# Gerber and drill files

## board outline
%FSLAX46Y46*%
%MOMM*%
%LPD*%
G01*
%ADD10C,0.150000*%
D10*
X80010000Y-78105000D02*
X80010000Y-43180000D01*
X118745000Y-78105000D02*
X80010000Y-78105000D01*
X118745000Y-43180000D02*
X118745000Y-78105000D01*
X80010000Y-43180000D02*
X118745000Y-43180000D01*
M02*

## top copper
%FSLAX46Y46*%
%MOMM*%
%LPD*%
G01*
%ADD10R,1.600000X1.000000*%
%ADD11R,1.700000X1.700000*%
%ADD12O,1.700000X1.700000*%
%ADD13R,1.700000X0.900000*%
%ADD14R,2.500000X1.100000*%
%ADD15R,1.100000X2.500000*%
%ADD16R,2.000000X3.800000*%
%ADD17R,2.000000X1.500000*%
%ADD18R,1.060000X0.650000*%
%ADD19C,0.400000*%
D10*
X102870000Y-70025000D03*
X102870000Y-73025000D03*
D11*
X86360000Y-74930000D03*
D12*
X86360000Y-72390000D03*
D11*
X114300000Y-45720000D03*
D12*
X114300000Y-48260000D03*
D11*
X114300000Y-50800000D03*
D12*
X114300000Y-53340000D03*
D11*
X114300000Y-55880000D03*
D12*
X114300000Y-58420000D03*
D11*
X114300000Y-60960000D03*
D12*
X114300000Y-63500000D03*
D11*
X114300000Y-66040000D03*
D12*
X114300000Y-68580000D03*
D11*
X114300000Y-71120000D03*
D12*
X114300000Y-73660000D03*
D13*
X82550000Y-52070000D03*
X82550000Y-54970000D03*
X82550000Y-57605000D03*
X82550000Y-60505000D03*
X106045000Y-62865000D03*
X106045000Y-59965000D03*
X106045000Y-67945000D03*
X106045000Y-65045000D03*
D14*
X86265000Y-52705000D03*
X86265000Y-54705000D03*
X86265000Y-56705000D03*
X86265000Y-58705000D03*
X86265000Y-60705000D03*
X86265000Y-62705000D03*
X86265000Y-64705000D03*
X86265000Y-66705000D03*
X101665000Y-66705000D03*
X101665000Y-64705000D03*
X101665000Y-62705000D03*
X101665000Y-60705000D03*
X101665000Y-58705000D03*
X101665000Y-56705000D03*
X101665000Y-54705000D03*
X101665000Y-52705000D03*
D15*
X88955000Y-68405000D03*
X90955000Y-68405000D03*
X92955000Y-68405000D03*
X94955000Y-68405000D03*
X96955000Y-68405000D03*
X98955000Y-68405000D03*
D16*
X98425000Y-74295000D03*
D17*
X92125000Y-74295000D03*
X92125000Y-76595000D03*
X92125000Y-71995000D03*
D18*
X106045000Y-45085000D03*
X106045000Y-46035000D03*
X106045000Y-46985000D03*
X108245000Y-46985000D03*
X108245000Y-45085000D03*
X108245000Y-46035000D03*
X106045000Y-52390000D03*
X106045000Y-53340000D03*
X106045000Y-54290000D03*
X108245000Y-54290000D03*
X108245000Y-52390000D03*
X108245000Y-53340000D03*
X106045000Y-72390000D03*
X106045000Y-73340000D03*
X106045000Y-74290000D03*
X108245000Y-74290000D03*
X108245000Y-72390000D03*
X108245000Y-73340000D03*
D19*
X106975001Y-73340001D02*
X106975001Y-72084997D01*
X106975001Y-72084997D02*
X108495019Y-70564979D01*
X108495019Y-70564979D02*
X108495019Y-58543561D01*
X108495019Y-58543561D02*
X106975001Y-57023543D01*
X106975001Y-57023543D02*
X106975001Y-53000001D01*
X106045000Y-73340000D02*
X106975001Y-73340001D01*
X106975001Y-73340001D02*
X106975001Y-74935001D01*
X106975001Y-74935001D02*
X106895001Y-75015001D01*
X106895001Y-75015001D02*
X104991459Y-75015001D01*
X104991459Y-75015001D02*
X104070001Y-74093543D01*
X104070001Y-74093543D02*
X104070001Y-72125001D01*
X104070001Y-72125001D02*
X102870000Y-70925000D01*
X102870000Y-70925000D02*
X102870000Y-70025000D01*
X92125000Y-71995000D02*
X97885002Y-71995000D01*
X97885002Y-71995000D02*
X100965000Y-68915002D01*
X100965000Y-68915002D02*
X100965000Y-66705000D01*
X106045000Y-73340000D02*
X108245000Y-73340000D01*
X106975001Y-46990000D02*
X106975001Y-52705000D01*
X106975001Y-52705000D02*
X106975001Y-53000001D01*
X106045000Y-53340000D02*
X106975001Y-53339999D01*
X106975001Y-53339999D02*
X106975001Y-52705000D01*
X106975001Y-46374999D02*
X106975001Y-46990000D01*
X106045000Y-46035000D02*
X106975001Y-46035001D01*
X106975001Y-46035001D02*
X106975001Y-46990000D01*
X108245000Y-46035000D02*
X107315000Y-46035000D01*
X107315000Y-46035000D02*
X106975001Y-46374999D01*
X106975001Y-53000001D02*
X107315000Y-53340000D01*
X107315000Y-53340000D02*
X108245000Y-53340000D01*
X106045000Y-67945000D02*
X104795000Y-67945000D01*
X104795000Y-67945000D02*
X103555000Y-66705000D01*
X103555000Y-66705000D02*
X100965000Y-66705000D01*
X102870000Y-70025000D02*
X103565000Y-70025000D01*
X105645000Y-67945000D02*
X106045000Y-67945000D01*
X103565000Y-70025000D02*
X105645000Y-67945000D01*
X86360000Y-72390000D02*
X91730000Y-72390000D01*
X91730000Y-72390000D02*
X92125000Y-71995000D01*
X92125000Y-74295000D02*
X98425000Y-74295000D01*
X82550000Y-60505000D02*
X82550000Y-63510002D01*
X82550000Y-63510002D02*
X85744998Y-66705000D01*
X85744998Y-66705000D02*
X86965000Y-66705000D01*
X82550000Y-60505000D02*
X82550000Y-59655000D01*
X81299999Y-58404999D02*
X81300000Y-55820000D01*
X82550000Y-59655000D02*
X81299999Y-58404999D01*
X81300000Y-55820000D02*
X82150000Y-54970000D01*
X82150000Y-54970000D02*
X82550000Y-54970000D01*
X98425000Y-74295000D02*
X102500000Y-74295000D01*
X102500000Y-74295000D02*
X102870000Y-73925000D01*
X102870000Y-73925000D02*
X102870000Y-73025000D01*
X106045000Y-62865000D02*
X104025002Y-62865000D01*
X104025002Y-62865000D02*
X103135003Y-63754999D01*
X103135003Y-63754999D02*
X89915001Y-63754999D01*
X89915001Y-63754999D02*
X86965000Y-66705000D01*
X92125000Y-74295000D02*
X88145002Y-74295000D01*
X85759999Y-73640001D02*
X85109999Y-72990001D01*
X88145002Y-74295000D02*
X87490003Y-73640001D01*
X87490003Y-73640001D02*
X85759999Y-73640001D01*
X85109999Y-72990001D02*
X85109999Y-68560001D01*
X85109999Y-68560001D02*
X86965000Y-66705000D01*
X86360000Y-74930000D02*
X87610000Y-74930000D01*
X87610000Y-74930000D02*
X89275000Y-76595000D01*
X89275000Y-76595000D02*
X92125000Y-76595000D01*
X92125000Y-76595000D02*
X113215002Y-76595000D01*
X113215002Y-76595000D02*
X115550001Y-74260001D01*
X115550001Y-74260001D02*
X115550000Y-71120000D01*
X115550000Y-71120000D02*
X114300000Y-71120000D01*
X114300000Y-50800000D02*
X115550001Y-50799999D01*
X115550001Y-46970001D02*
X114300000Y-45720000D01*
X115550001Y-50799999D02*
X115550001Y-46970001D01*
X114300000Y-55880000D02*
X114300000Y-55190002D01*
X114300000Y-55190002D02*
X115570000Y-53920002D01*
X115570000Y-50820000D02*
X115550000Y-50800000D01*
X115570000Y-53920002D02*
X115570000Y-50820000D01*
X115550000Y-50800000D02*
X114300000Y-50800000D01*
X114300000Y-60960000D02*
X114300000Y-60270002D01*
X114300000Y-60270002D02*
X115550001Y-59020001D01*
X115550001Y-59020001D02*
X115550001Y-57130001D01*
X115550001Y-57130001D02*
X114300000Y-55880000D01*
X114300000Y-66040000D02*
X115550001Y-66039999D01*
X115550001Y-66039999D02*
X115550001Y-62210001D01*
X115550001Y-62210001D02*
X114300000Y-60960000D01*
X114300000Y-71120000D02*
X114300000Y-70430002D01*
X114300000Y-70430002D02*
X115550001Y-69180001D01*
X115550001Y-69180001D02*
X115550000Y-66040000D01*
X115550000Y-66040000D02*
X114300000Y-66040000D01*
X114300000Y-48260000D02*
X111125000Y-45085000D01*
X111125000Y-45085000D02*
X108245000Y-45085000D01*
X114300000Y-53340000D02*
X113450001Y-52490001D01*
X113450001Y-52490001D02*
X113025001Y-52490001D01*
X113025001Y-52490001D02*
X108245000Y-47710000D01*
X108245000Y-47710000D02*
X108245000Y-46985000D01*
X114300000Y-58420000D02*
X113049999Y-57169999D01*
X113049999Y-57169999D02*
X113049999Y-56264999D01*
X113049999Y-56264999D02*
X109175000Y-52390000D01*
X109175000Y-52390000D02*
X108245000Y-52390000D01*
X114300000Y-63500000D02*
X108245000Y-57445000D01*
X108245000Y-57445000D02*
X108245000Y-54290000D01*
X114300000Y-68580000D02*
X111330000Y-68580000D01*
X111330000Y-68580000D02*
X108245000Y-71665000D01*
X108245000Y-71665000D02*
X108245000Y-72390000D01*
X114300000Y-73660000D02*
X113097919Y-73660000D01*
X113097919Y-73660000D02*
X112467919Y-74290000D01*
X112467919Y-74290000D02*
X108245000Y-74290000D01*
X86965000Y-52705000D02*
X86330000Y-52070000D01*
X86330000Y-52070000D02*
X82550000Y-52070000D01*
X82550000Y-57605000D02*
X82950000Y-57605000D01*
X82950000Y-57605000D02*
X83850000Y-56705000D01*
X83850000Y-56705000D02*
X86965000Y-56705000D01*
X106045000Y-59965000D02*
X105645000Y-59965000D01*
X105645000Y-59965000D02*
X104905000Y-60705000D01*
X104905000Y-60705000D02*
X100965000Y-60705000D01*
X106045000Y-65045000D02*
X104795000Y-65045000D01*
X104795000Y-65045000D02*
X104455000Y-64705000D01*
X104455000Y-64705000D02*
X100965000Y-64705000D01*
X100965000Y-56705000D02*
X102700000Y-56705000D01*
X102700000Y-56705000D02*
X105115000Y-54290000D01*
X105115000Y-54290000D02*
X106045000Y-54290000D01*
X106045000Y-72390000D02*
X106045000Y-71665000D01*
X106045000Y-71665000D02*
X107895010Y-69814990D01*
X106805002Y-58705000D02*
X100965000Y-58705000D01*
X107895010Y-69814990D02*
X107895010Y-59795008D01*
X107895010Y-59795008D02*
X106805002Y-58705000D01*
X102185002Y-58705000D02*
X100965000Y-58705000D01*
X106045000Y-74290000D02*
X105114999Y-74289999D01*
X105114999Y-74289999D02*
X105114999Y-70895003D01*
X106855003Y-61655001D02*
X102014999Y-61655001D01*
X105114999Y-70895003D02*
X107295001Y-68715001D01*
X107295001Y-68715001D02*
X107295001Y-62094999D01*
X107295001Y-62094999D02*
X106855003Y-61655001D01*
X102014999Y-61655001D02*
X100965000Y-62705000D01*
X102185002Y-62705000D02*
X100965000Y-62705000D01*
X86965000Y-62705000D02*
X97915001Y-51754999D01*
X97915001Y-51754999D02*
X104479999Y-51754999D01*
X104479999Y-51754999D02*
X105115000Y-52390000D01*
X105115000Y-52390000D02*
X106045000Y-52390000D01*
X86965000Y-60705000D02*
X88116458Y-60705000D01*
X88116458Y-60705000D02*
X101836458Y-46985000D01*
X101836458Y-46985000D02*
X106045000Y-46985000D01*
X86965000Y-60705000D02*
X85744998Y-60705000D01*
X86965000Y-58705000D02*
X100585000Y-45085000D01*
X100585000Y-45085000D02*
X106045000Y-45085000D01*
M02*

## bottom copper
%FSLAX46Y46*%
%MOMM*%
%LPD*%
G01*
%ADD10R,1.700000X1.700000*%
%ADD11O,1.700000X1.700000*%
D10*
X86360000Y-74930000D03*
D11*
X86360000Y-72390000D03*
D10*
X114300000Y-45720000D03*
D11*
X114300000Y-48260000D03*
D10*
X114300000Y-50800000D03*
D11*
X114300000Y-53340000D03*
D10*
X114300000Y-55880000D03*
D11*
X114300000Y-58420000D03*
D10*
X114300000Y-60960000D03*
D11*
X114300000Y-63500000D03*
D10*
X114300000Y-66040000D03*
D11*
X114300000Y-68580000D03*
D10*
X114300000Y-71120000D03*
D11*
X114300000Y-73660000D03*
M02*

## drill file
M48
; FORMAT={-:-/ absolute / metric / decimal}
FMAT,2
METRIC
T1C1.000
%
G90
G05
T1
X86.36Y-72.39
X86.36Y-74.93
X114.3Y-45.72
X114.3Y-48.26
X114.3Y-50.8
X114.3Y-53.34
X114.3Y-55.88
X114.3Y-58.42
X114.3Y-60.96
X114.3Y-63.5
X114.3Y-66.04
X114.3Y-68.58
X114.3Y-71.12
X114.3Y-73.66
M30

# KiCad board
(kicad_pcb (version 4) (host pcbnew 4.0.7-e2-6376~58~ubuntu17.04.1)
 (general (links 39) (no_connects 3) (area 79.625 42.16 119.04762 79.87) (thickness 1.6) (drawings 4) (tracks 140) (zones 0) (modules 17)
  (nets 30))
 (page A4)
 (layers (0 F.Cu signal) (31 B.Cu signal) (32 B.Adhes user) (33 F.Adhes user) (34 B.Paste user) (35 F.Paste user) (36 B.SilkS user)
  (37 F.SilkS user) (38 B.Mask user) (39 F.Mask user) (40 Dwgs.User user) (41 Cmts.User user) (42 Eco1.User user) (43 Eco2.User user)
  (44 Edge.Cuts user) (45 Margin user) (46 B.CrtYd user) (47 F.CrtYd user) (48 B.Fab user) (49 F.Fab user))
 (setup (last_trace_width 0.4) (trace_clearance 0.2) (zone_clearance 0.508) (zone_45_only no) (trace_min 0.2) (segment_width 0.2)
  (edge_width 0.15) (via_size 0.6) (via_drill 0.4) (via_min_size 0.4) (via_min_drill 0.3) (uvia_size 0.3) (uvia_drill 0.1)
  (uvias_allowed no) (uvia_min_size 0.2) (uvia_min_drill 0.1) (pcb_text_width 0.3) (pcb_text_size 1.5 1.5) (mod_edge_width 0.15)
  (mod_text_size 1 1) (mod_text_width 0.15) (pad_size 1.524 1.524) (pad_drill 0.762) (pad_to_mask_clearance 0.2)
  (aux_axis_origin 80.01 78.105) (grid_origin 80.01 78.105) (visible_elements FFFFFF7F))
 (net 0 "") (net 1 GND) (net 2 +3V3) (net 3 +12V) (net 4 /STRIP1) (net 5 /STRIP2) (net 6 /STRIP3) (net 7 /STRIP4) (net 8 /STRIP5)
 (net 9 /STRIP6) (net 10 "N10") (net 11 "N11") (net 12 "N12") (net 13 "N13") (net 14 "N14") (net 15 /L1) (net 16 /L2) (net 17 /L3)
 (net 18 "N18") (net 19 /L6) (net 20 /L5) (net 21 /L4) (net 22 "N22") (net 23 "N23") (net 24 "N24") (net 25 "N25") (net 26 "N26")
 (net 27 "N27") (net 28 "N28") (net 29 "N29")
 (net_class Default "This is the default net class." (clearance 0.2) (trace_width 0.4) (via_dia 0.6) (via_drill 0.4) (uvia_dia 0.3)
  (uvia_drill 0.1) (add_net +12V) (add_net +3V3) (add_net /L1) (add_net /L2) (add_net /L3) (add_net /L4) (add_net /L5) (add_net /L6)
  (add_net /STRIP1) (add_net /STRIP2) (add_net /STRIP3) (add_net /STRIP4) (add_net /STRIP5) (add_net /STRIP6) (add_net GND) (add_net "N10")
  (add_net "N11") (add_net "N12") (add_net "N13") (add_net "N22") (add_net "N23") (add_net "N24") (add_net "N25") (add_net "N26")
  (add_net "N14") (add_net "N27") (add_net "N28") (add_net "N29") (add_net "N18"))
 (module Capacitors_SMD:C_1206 (layer F.Cu) (at 102.87 71.525 270)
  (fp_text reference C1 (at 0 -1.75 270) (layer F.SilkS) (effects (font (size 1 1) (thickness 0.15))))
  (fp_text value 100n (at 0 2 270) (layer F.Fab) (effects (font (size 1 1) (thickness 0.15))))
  (pad 1 smd rect (at -1.5 0 270) (size 1 1.6) (layers F.Cu F.Paste F.Mask) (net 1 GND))
  (pad 2 smd rect (at 1.5 0 270) (size 1 1.6) (layers F.Cu F.Paste F.Mask) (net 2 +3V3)))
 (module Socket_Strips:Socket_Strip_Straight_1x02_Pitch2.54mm (layer F.Cu) (at 86.36 74.93 180)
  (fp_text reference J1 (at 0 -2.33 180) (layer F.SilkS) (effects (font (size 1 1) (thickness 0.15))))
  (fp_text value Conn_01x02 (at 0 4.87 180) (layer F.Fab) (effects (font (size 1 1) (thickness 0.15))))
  (pad 1 thru_hole rect (at 0 0 180) (size 1.7 1.7) (drill 1) (layers *.Cu *.Mask) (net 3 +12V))
  (pad 2 thru_hole oval (at 0 2.54 180) (size 1.7 1.7) (drill 1) (layers *.Cu *.Mask) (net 1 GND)))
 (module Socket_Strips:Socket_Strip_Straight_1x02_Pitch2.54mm (layer F.Cu) (at 114.3 45.72)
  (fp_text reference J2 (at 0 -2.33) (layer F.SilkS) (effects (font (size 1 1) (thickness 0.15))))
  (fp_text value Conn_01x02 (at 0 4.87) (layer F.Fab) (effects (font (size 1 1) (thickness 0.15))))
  (pad 1 thru_hole rect (at 0 0) (size 1.7 1.7) (drill 1) (layers *.Cu *.Mask) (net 3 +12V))
  (pad 2 thru_hole oval (at 0 2.54) (size 1.7 1.7) (drill 1) (layers *.Cu *.Mask) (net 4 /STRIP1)))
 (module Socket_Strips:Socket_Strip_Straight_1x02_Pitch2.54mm (layer F.Cu) (at 114.3 50.8)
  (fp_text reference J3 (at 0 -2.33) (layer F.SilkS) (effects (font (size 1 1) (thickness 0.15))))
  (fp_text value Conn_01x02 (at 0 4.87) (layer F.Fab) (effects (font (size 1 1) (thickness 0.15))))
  (pad 1 thru_hole rect (at 0 0) (size 1.7 1.7) (drill 1) (layers *.Cu *.Mask) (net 3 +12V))
  (pad 2 thru_hole oval (at 0 2.54) (size 1.7 1.7) (drill 1) (layers *.Cu *.Mask) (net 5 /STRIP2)))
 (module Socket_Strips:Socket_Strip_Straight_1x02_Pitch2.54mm (layer F.Cu) (at 114.3 55.88)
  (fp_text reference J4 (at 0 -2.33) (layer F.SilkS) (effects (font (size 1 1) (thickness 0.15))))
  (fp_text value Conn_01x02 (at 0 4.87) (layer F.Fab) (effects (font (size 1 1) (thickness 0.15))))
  (pad 1 thru_hole rect (at 0 0) (size 1.7 1.7) (drill 1) (layers *.Cu *.Mask) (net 3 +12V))
  (pad 2 thru_hole oval (at 0 2.54) (size 1.7 1.7) (drill 1) (layers *.Cu *.Mask) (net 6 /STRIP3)))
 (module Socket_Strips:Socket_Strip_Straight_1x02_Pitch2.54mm (layer F.Cu) (at 114.3 60.96)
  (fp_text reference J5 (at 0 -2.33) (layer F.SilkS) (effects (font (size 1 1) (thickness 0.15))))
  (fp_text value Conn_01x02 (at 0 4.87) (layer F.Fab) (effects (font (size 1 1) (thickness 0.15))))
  (pad 1 thru_hole rect (at 0 0) (size 1.7 1.7) (drill 1) (layers *.Cu *.Mask) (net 3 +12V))
  (pad 2 thru_hole oval (at 0 2.54) (size 1.7 1.7) (drill 1) (layers *.Cu *.Mask) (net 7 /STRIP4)))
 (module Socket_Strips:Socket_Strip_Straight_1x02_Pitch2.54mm (layer F.Cu) (at 114.3 66.04)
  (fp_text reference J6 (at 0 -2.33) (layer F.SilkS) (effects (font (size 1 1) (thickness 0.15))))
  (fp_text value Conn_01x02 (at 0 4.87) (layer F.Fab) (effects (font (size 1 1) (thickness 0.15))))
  (pad 1 thru_hole rect (at 0 0) (size 1.7 1.7) (drill 1) (layers *.Cu *.Mask) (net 3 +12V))
  (pad 2 thru_hole oval (at 0 2.54) (size 1.7 1.7) (drill 1) (layers *.Cu *.Mask) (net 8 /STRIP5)))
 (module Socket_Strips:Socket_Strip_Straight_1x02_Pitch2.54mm (layer F.Cu) (at 114.3 71.12)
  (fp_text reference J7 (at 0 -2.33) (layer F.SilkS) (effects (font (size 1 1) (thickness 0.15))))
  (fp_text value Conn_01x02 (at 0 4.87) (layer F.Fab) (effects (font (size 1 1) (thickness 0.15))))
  (pad 1 thru_hole rect (at 0 0) (size 1.7 1.7) (drill 1) (layers *.Cu *.Mask) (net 3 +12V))
  (pad 2 thru_hole oval (at 0 2.54) (size 1.7 1.7) (drill 1) (layers *.Cu *.Mask) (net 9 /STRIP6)))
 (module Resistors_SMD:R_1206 (layer F.Cu) (at 82.55 53.52 270)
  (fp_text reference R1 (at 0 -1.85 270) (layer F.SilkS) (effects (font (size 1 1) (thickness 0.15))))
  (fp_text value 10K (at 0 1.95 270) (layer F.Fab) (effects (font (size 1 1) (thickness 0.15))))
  (pad 1 smd rect (at -1.45 0 270) (size 0.9 1.7) (layers F.Cu F.Paste F.Mask) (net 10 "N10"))
  (pad 2 smd rect (at 1.45 0 270) (size 0.9 1.7) (layers F.Cu F.Paste F.Mask) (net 2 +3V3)))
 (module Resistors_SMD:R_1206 (layer F.Cu) (at 82.55 59.055 270)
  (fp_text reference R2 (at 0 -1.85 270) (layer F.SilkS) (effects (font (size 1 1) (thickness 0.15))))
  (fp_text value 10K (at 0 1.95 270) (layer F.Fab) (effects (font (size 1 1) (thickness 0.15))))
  (pad 1 smd rect (at -1.45 0 270) (size 0.9 1.7) (layers F.Cu F.Paste F.Mask) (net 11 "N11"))
  (pad 2 smd rect (at 1.45 0 270) (size 0.9 1.7) (layers F.Cu F.Paste F.Mask) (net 2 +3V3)))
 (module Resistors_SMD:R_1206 (layer F.Cu) (at 106.045 61.415 90)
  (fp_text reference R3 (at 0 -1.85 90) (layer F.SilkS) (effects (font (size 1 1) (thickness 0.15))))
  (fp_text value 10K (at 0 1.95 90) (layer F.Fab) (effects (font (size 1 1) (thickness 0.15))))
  (pad 1 smd rect (at -1.45 0 90) (size 0.9 1.7) (layers F.Cu F.Paste F.Mask) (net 2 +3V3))
  (pad 2 smd rect (at 1.45 0 90) (size 0.9 1.7) (layers F.Cu F.Paste F.Mask) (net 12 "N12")))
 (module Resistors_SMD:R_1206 (layer F.Cu) (at 106.045 66.495 90)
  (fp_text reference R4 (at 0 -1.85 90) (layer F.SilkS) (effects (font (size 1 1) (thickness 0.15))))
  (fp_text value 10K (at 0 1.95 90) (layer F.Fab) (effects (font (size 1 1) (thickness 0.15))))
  (pad 1 smd rect (at -1.45 0 90) (size 0.9 1.7) (layers F.Cu F.Paste F.Mask) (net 1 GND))
  (pad 2 smd rect (at 1.45 0 90) (size 0.9 1.7) (layers F.Cu F.Paste F.Mask) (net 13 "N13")))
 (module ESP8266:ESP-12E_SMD (layer F.Cu) (at 86.965 52.705)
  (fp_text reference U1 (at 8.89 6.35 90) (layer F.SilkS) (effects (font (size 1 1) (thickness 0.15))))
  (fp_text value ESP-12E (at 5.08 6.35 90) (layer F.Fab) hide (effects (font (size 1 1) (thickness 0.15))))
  (pad 1 smd rect (at 0 0) (size 2.5 1.1) (drill (offset -0.7 0)) (layers F.Cu F.Paste F.Mask) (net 10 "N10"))
  (pad 2 smd rect (at 0 2) (size 2.5 1.1) (drill (offset -0.7 0)) (layers F.Cu F.Paste F.Mask) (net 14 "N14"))
  (pad 3 smd rect (at 0 4) (size 2.5 1.1) (drill (offset -0.7 0)) (layers F.Cu F.Paste F.Mask) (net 11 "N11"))
  (pad 4 smd rect (at 0 6) (size 2.5 1.1) (drill (offset -0.7 0)) (layers F.Cu F.Paste F.Mask) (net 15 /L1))
  (pad 5 smd rect (at 0 8) (size 2.5 1.1) (drill (offset -0.7 0)) (layers F.Cu F.Paste F.Mask) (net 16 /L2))
  (pad 6 smd rect (at 0 10) (size 2.5 1.1) (drill (offset -0.7 0)) (layers F.Cu F.Paste F.Mask) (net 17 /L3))
  (pad 7 smd rect (at 0 12) (size 2.5 1.1) (drill (offset -0.7 0)) (layers F.Cu F.Paste F.Mask) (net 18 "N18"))
  (pad 8 smd rect (at 0 14) (size 2.5 1.1) (drill (offset -0.7 0)) (layers F.Cu F.Paste F.Mask) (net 2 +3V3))
  (pad 9 smd rect (at 14 14) (size 2.5 1.1) (drill (offset 0.7 0)) (layers F.Cu F.Paste F.Mask) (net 1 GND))
  (pad 10 smd rect (at 14 12) (size 2.5 1.1) (drill (offset 0.7 0)) (layers F.Cu F.Paste F.Mask) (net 13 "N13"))
  (pad 11 smd rect (at 14 10) (size 2.5 1.1) (drill (offset 0.7 0)) (layers F.Cu F.Paste F.Mask) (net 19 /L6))
  (pad 12 smd rect (at 14 8) (size 2.5 1.1) (drill (offset 0.7 0)) (layers F.Cu F.Paste F.Mask) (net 12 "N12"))
  (pad 13 smd rect (at 14 6) (size 2.5 1.1) (drill (offset 0.7 0)) (layers F.Cu F.Paste F.Mask) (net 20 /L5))
  (pad 14 smd rect (at 14 4) (size 2.5 1.1) (drill (offset 0.7 0)) (layers F.Cu F.Paste F.Mask) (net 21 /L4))
  (pad 15 smd rect (at 14 2) (size 2.5 1.1) (drill (offset 0.7 0)) (layers F.Cu F.Paste F.Mask) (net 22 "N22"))
  (pad 16 smd rect (at 14 0) (size 2.5 1.1) (drill (offset 0.7 0)) (layers F.Cu F.Paste F.Mask) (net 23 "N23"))
  (pad 17 smd rect (at 1.99 15 90) (size 2.5 1.1) (drill (offset -0.7 0)) (layers F.Cu F.Paste F.Mask) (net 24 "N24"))
  (pad 18 smd rect (at 3.99 15 90) (size 2.5 1.1) (drill (offset -0.7 0)) (layers F.Cu F.Paste F.Mask) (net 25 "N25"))
  (pad 19 smd rect (at 5.99 15 90) (size 2.5 1.1) (drill (offset -0.7 0)) (layers F.Cu F.Paste F.Mask) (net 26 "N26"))
  (pad 20 smd rect (at 7.99 15 90) (size 2.5 1.1) (drill (offset -0.7 0)) (layers F.Cu F.Paste F.Mask) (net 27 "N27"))
  (pad 21 smd rect (at 9.99 15 90) (size 2.5 1.1) (drill (offset -0.7 0)) (layers F.Cu F.Paste F.Mask) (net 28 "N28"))
  (pad 22 smd rect (at 11.99 15 90) (size 2.5 1.1) (drill (offset -0.7 0)) (layers F.Cu F.Paste F.Mask) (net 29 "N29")))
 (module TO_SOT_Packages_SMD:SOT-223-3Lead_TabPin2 (layer F.Cu) (at 95.275 74.295)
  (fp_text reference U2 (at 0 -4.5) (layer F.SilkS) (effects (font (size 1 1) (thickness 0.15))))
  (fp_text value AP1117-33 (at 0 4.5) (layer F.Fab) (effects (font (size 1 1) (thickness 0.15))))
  (pad 2 smd rect (at 3.15 0) (size 2 3.8) (layers F.Cu F.Paste F.Mask) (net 2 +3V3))
  (pad 2 smd rect (at -3.15 0) (size 2 1.5) (layers F.Cu F.Paste F.Mask) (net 2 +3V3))
  (pad 3 smd rect (at -3.15 2.3) (size 2 1.5) (layers F.Cu F.Paste F.Mask) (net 3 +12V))
  (pad 1 smd rect (at -3.15 -2.3) (size 2 1.5) (layers F.Cu F.Paste F.Mask) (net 1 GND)))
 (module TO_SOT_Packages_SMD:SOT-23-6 (layer F.Cu) (at 107.145 46.035)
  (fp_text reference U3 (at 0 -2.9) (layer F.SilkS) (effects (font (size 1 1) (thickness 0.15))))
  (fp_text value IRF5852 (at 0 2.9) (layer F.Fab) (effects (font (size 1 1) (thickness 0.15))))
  (pad 1 smd rect (at -1.1 -0.95) (size 1.06 0.65) (layers F.Cu F.Paste F.Mask) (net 15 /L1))
  (pad 2 smd rect (at -1.1 0) (size 1.06 0.65) (layers F.Cu F.Paste F.Mask) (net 1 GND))
  (pad 3 smd rect (at -1.1 0.95) (size 1.06 0.65) (layers F.Cu F.Paste F.Mask) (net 16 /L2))
  (pad 4 smd rect (at 1.1 0.95) (size 1.06 0.65) (layers F.Cu F.Paste F.Mask) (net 5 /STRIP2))
  (pad 6 smd rect (at 1.1 -0.95) (size 1.06 0.65) (layers F.Cu F.Paste F.Mask) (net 4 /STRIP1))
  (pad 5 smd rect (at 1.1 0) (size 1.06 0.65) (layers F.Cu F.Paste F.Mask) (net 1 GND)))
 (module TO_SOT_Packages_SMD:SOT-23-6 (layer F.Cu) (at 107.145 53.34)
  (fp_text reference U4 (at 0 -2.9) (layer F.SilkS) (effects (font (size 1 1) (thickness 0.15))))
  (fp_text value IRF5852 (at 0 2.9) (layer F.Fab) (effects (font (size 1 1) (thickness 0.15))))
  (pad 1 smd rect (at -1.1 -0.95) (size 1.06 0.65) (layers F.Cu F.Paste F.Mask) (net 17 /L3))
  (pad 2 smd rect (at -1.1 0) (size 1.06 0.65) (layers F.Cu F.Paste F.Mask) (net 1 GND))
  (pad 3 smd rect (at -1.1 0.95) (size 1.06 0.65) (layers F.Cu F.Paste F.Mask) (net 21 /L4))
  (pad 4 smd rect (at 1.1 0.95) (size 1.06 0.65) (layers F.Cu F.Paste F.Mask) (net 7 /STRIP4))
  (pad 6 smd rect (at 1.1 -0.95) (size 1.06 0.65) (layers F.Cu F.Paste F.Mask) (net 6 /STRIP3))
  (pad 5 smd rect (at 1.1 0) (size 1.06 0.65) (layers F.Cu F.Paste F.Mask) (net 1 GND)))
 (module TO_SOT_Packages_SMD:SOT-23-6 (layer F.Cu) (at 107.145 73.34)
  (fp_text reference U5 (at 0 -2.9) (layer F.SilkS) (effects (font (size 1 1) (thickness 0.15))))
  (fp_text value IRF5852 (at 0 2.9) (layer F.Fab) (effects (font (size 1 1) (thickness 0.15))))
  (pad 1 smd rect (at -1.1 -0.95) (size 1.06 0.65) (layers F.Cu F.Paste F.Mask) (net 20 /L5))
  (pad 2 smd rect (at -1.1 0) (size 1.06 0.65) (layers F.Cu F.Paste F.Mask) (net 1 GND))
  (pad 3 smd rect (at -1.1 0.95) (size 1.06 0.65) (layers F.Cu F.Paste F.Mask) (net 19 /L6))
  (pad 4 smd rect (at 1.1 0.95) (size 1.06 0.65) (layers F.Cu F.Paste F.Mask) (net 9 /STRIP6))
  (pad 6 smd rect (at 1.1 -0.95) (size 1.06 0.65) (layers F.Cu F.Paste F.Mask) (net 8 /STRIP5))
  (pad 5 smd rect (at 1.1 0) (size 1.06 0.65) (layers F.Cu F.Paste F.Mask) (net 1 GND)))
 (gr_line (start 80.01 78.105) (end 80.01 43.18) (layer Edge.Cuts) (width 0.15))
 (gr_line (start 118.745 78.105) (end 80.01 78.105) (layer Edge.Cuts) (width 0.15))
 (gr_line (start 118.745 43.18) (end 118.745 78.105) (layer Edge.Cuts) (width 0.15))
 (gr_line (start 80.01 43.18) (end 118.745 43.18) (layer Edge.Cuts) (width 0.15))
 (segment (start 106.975001 73.340001) (end 106.975001 72.084997) (width 0.4) (layer F.Cu) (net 1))
 (segment (start 106.975001 72.084997) (end 108.495019 70.564979) (width 0.4) (layer F.Cu) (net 1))
 (segment (start 108.495019 70.564979) (end 108.495019 58.543561) (width 0.4) (layer F.Cu) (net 1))
 (segment (start 108.495019 58.543561) (end 106.975001 57.023543) (width 0.4) (layer F.Cu) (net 1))
 (segment (start 106.975001 57.023543) (end 106.975001 53.000001) (width 0.4) (layer F.Cu) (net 1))
 (segment (start 106.045 73.34) (end 106.975001 73.340001) (width 0.4) (layer F.Cu) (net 1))
 (segment (start 106.975001 73.340001) (end 106.975001 74.935001) (width 0.4) (layer F.Cu) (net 1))
 (segment (start 106.975001 74.935001) (end 106.895001 75.015001) (width 0.4) (layer F.Cu) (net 1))
 (segment (start 106.895001 75.015001) (end 104.991459 75.015001) (width 0.4) (layer F.Cu) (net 1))
 (segment (start 104.991459 75.015001) (end 104.070001 74.093543) (width 0.4) (layer F.Cu) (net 1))
 (segment (start 104.070001 74.093543) (end 104.070001 72.125001) (width 0.4) (layer F.Cu) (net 1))
 (segment (start 104.070001 72.125001) (end 102.87 70.925) (width 0.4) (layer F.Cu) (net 1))
 (segment (start 102.87 70.925) (end 102.87 70.025) (width 0.4) (layer F.Cu) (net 1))
 (segment (start 92.125 71.995) (end 97.885002 71.995) (width 0.4) (layer F.Cu) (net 1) (status 10))
 (segment (start 97.885002 71.995) (end 100.965 68.915002) (width 0.4) (layer F.Cu) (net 1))
 (segment (start 100.965 68.915002) (end 100.965 66.705) (width 0.4) (layer F.Cu) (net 1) (status 20))
 (segment (start 106.045 73.34) (end 108.245 73.34) (width 0.4) (layer F.Cu) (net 1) (status 30))
 (segment (start 106.975001 46.99) (end 106.975001 52.705) (width 0.4) (layer F.Cu) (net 1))
 (segment (start 106.975001 52.705) (end 106.975001 53.000001) (width 0.4) (layer F.Cu) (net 1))
 (segment (start 106.045 53.34) (end 106.975001 53.339999) (width 0.4) (layer F.Cu) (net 1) (status 10))
 (segment (start 106.975001 53.339999) (end 106.975001 52.705) (width 0.4) (layer F.Cu) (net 1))
 (segment (start 106.975001 46.374999) (end 106.975001 46.99) (width 0.4) (layer F.Cu) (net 1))
 (segment (start 106.045 46.035) (end 106.975001 46.035001) (width 0.4) (layer F.Cu) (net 1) (status 10))
 (segment (start 106.975001 46.035001) (end 106.975001 46.99) (width 0.4) (layer F.Cu) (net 1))
 (segment (start 108.245 46.035) (end 107.315 46.035) (width 0.4) (layer F.Cu) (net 1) (status 10))
 (segment (start 107.315 46.035) (end 106.975001 46.374999) (width 0.4) (layer F.Cu) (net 1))
 (segment (start 106.975001 53.000001) (end 107.315 53.34) (width 0.4) (layer F.Cu) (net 1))
 (segment (start 107.315 53.34) (end 108.245 53.34) (width 0.4) (layer F.Cu) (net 1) (status 20))
 (segment (start 106.045 67.945) (end 104.795 67.945) (width 0.4) (layer F.Cu) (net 1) (status 10))
 (segment (start 104.795 67.945) (end 103.555 66.705) (width 0.4) (layer F.Cu) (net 1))
 (segment (start 103.555 66.705) (end 100.965 66.705) (width 0.4) (layer F.Cu) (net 1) (status 20))
 (segment (start 102.87 70.025) (end 103.565 70.025) (width 0.4) (layer F.Cu) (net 1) (status 30))
 (segment (start 105.645 67.945) (end 106.045 67.945) (width 0.4) (layer F.Cu) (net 1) (status 30))
 (segment (start 103.565 70.025) (end 105.645 67.945) (width 0.4) (layer F.Cu) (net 1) (status 30))
 (segment (start 86.36 72.39) (end 91.73 72.39) (width 0.4) (layer F.Cu) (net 1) (status 30))
 (segment (start 91.73 72.39) (end 92.125 71.995) (width 0.4) (layer F.Cu) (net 1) (status 30))
 (segment (start 92.125 74.295) (end 98.425 74.295) (width 0.4) (layer F.Cu) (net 2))
 (segment (start 82.55 60.505) (end 82.55 63.510002) (width 0.4) (layer F.Cu) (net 2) (status 10))
 (segment (start 82.55 63.510002) (end 85.744998 66.705) (width 0.4) (layer F.Cu) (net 2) (status 20))
 (segment (start 85.744998 66.705) (end 86.965 66.705) (width 0.4) (layer F.Cu) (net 2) (status 30))
 (segment (start 82.55 60.505) (end 82.55 59.655) (width 0.4) (layer F.Cu) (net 2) (status 10))
 (segment (start 81.299999 58.404999) (end 81.3 55.82) (width 0.4) (layer F.Cu) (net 2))
 (segment (start 82.55 59.655) (end 81.299999 58.404999) (width 0.4) (layer F.Cu) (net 2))
 (segment (start 81.3 55.82) (end 82.15 54.97) (width 0.4) (layer F.Cu) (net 2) (status 20))
 (segment (start 82.15 54.97) (end 82.55 54.97) (width 0.4) (layer F.Cu) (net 2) (status 30))
 (segment (start 98.425 74.295) (end 102.5 74.295) (width 0.4) (layer F.Cu) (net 2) (status 10))
 (segment (start 102.5 74.295) (end 102.87 73.925) (width 0.4) (layer F.Cu) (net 2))
 (segment (start 102.87 73.925) (end 102.87 73.025) (width 0.4) (layer F.Cu) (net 2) (status 20))
 (segment (start 106.045 62.865) (end 104.025002 62.865) (width 0.4) (layer F.Cu) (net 2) (status 10))
 (segment (start 104.025002 62.865) (end 103.135003 63.754999) (width 0.4) (layer F.Cu) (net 2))
 (segment (start 103.135003 63.754999) (end 89.915001 63.754999) (width 0.4) (layer F.Cu) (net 2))
 (segment (start 89.915001 63.754999) (end 86.965 66.705) (width 0.4) (layer F.Cu) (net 2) (status 20))
 (segment (start 92.125 74.295) (end 88.145002 74.295) (width 0.4) (layer F.Cu) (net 2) (status 10))
 (segment (start 85.759999 73.640001) (end 85.109999 72.990001) (width 0.4) (layer F.Cu) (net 2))
 (segment (start 88.145002 74.295) (end 87.490003 73.640001) (width 0.4) (layer F.Cu) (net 2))
 (segment (start 87.490003 73.640001) (end 85.759999 73.640001) (width 0.4) (layer F.Cu) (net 2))
 (segment (start 85.109999 72.990001) (end 85.109999 68.560001) (width 0.4) (layer F.Cu) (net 2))
 (segment (start 85.109999 68.560001) (end 86.965 66.705) (width 0.4) (layer F.Cu) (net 2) (status 20))
 (segment (start 86.36 74.93) (end 87.61 74.93) (width 0.4) (layer F.Cu) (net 3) (status 10))
 (segment (start 87.61 74.93) (end 89.275 76.595) (width 0.4) (layer F.Cu) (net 3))
 (segment (start 89.275 76.595) (end 92.125 76.595) (width 0.4) (layer F.Cu) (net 3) (status 20))
 (segment (start 92.125 76.595) (end 113.215002 76.595) (width 0.4) (layer F.Cu) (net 3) (status 10))
 (segment (start 113.215002 76.595) (end 115.550001 74.260001) (width 0.4) (layer F.Cu) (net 3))
 (segment (start 115.550001 74.260001) (end 115.55 71.12) (width 0.4) (layer F.Cu) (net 3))
 (segment (start 115.55 71.12) (end 114.3 71.12) (width 0.4) (layer F.Cu) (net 3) (status 20))
 (segment (start 114.3 50.8) (end 115.550001 50.799999) (width 0.4) (layer F.Cu) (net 3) (status 10))
 (segment (start 115.550001 46.970001) (end 114.3 45.72) (width 0.4) (layer F.Cu) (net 3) (status 20))
 (segment (start 115.550001 50.799999) (end 115.550001 46.970001) (width 0.4) (layer F.Cu) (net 3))
 (segment (start 114.3 55.88) (end 114.3 55.190002) (width 0.4) (layer F.Cu) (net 3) (status 30))
 (segment (start 114.3 55.190002) (end 115.57 53.920002) (width 0.4) (layer F.Cu) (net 3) (status 10))
 (segment (start 115.57 50.82) (end 115.55 50.8) (width 0.4) (layer F.Cu) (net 3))
 (segment (start 115.57 53.920002) (end 115.57 50.82) (width 0.4) (layer F.Cu) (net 3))
 (segment (start 115.55 50.8) (end 114.3 50.8) (width 0.4) (layer F.Cu) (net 3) (status 20))
 (segment (start 114.3 60.96) (end 114.3 60.270002) (width 0.4) (layer F.Cu) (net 3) (status 30))
 (segment (start 114.3 60.270002) (end 115.550001 59.020001) (width 0.4) (layer F.Cu) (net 3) (status 10))
 (segment (start 115.550001 59.020001) (end 115.550001 57.130001) (width 0.4) (layer F.Cu) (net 3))
 (segment (start 115.550001 57.130001) (end 114.3 55.88) (width 0.4) (layer F.Cu) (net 3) (status 20))
 (segment (start 114.3 66.04) (end 115.550001 66.039999) (width 0.4) (layer F.Cu) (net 3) (status 10))
 (segment (start 115.550001 66.039999) (end 115.550001 62.210001) (width 0.4) (layer F.Cu) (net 3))
 (segment (start 115.550001 62.210001) (end 114.3 60.96) (width 0.4) (layer F.Cu) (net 3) (status 20))
 (segment (start 114.3 71.12) (end 114.3 70.430002) (width 0.4) (layer F.Cu) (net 3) (status 30))
 (segment (start 114.3 70.430002) (end 115.550001 69.180001) (width 0.4) (layer F.Cu) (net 3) (status 10))
 (segment (start 115.550001 69.180001) (end 115.55 66.04) (width 0.4) (layer F.Cu) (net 3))
 (segment (start 115.55 66.04) (end 114.3 66.04) (width 0.4) (layer F.Cu) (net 3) (status 20))
 (segment (start 114.3 48.26) (end 111.125 45.085) (width 0.4) (layer F.Cu) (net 4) (status 10))
 (segment (start 111.125 45.085) (end 108.245 45.085) (width 0.4) (layer F.Cu) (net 4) (status 20))
 (segment (start 114.3 53.34) (end 113.450001 52.490001) (width 0.4) (layer F.Cu) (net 5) (status 10))
 (segment (start 113.450001 52.490001) (end 113.025001 52.490001) (width 0.4) (layer F.Cu) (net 5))
 (segment (start 113.025001 52.490001) (end 108.245 47.71) (width 0.4) (layer F.Cu) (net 5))
 (segment (start 108.245 47.71) (end 108.245 46.985) (width 0.4) (layer F.Cu) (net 5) (status 20))
 (segment (start 114.3 58.42) (end 113.049999 57.169999) (width 0.4) (layer F.Cu) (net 6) (status 10))
 (segment (start 113.049999 57.169999) (end 113.049999 56.264999) (width 0.4) (layer F.Cu) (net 6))
 (segment (start 113.049999 56.264999) (end 109.175 52.39) (width 0.4) (layer F.Cu) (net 6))
 (segment (start 109.175 52.39) (end 108.245 52.39) (width 0.4) (layer F.Cu) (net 6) (status 20))
 (segment (start 114.3 63.5) (end 108.245 57.445) (width 0.4) (layer F.Cu) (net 7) (status 10))
 (segment (start 108.245 57.445) (end 108.245 54.29) (width 0.4) (layer F.Cu) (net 7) (status 20))
 (segment (start 114.3 68.58) (end 111.33 68.58) (width 0.4) (layer F.Cu) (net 8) (status 10))
 (segment (start 111.33 68.58) (end 108.245 71.665) (width 0.4) (layer F.Cu) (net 8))
 (segment (start 108.245 71.665) (end 108.245 72.39) (width 0.4) (layer F.Cu) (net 8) (status 20))
 (segment (start 114.3 73.66) (end 113.097919 73.66) (width 0.4) (layer F.Cu) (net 9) (status 10))
 (segment (start 113.097919 73.66) (end 112.467919 74.29) (width 0.4) (layer F.Cu) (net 9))
 (segment (start 112.467919 74.29) (end 108.245 74.29) (width 0.4) (layer F.Cu) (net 9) (status 20))
 (segment (start 86.965 52.705) (end 86.33 52.07) (width 0.4) (layer F.Cu) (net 10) (status 10))
 (segment (start 86.33 52.07) (end 82.55 52.07) (width 0.4) (layer F.Cu) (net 10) (status 20))
 (segment (start 82.55 57.605) (end 82.95 57.605) (width 0.4) (layer F.Cu) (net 11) (status 30))
 (segment (start 82.95 57.605) (end 83.85 56.705) (width 0.4) (layer F.Cu) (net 11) (status 10))
 (segment (start 83.85 56.705) (end 86.965 56.705) (width 0.4) (layer F.Cu) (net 11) (status 20))
 (segment (start 106.045 59.965) (end 105.645 59.965) (width 0.4) (layer F.Cu) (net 12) (status 30))
 (segment (start 105.645 59.965) (end 104.905 60.705) (width 0.4) (layer F.Cu) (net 12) (status 10))
 (segment (start 104.905 60.705) (end 100.965 60.705) (width 0.4) (layer F.Cu) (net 12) (status 20))
 (segment (start 106.045 65.045) (end 104.795 65.045) (width 0.4) (layer F.Cu) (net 13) (status 10))
 (segment (start 104.795 65.045) (end 104.455 64.705) (width 0.4) (layer F.Cu) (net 13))
 (segment (start 104.455 64.705) (end 100.965 64.705) (width 0.4) (layer F.Cu) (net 13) (status 20))
 (segment (start 100.965 56.705) (end 102.7 56.705) (width 0.4) (layer F.Cu) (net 21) (status 30))
 (segment (start 102.7 56.705) (end 105.115 54.29) (width 0.4) (layer F.Cu) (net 21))
 (segment (start 105.115 54.29) (end 106.045 54.29) (width 0.4) (layer F.Cu) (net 21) (status 20))
 (segment (start 106.045 72.39) (end 106.045 71.665) (width 0.4) (layer F.Cu) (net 20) (status 10))
 (segment (start 106.045 71.665) (end 107.89501 69.81499) (width 0.4) (layer F.Cu) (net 20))
 (segment (start 106.805002 58.705) (end 100.965 58.705) (width 0.4) (layer F.Cu) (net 20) (status 20))
 (segment (start 107.89501 69.81499) (end 107.89501 59.795008) (width 0.4) (layer F.Cu) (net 20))
 (segment (start 107.89501 59.795008) (end 106.805002 58.705) (width 0.4) (layer F.Cu) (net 20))
 (segment (start 102.185002 58.705) (end 100.965 58.705) (width 0.4) (layer F.Cu) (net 20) (status 30))
 (segment (start 106.045 74.29) (end 105.114999 74.289999) (width 0.4) (layer F.Cu) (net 19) (status 10))
 (segment (start 105.114999 74.289999) (end 105.114999 70.895003) (width 0.4) (layer F.Cu) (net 19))
 (segment (start 106.855003 61.655001) (end 102.014999 61.655001) (width 0.4) (layer F.Cu) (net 19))
 (segment (start 105.114999 70.895003) (end 107.295001 68.715001) (width 0.4) (layer F.Cu) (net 19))
 (segment (start 107.295001 68.715001) (end 107.295001 62.094999) (width 0.4) (layer F.Cu) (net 19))
 (segment (start 107.295001 62.094999) (end 106.855003 61.655001) (width 0.4) (layer F.Cu) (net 19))
 (segment (start 102.014999 61.655001) (end 100.965 62.705) (width 0.4) (layer F.Cu) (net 19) (status 20))
 (segment (start 102.185002 62.705) (end 100.965 62.705) (width 0.4) (layer F.Cu) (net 19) (status 30))
 (segment (start 86.965 62.705) (end 97.915001 51.754999) (width 0.4) (layer F.Cu) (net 17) (status 10))
 (segment (start 97.915001 51.754999) (end 104.479999 51.754999) (width 0.4) (layer F.Cu) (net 17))
 (segment (start 104.479999 51.754999) (end 105.115 52.39) (width 0.4) (layer F.Cu) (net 17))
 (segment (start 105.115 52.39) (end 106.045 52.39) (width 0.4) (layer F.Cu) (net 17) (status 20))
 (segment (start 86.965 60.705) (end 88.116458 60.705) (width 0.4) (layer F.Cu) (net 16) (status 10))
 (segment (start 88.116458 60.705) (end 101.836458 46.985) (width 0.4) (layer F.Cu) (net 16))
 (segment (start 101.836458 46.985) (end 106.045 46.985) (width 0.4) (layer F.Cu) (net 16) (status 20))
 (segment (start 86.965 60.705) (end 85.744998 60.705) (width 0.4) (layer F.Cu) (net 16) (status 30))
 (segment (start 86.965 58.705) (end 100.585 45.085) (width 0.4) (layer F.Cu) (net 15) (status 10))
 (segment (start 100.585 45.085) (end 106.045 45.085) (width 0.4) (layer F.Cu) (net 15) (status 20)))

